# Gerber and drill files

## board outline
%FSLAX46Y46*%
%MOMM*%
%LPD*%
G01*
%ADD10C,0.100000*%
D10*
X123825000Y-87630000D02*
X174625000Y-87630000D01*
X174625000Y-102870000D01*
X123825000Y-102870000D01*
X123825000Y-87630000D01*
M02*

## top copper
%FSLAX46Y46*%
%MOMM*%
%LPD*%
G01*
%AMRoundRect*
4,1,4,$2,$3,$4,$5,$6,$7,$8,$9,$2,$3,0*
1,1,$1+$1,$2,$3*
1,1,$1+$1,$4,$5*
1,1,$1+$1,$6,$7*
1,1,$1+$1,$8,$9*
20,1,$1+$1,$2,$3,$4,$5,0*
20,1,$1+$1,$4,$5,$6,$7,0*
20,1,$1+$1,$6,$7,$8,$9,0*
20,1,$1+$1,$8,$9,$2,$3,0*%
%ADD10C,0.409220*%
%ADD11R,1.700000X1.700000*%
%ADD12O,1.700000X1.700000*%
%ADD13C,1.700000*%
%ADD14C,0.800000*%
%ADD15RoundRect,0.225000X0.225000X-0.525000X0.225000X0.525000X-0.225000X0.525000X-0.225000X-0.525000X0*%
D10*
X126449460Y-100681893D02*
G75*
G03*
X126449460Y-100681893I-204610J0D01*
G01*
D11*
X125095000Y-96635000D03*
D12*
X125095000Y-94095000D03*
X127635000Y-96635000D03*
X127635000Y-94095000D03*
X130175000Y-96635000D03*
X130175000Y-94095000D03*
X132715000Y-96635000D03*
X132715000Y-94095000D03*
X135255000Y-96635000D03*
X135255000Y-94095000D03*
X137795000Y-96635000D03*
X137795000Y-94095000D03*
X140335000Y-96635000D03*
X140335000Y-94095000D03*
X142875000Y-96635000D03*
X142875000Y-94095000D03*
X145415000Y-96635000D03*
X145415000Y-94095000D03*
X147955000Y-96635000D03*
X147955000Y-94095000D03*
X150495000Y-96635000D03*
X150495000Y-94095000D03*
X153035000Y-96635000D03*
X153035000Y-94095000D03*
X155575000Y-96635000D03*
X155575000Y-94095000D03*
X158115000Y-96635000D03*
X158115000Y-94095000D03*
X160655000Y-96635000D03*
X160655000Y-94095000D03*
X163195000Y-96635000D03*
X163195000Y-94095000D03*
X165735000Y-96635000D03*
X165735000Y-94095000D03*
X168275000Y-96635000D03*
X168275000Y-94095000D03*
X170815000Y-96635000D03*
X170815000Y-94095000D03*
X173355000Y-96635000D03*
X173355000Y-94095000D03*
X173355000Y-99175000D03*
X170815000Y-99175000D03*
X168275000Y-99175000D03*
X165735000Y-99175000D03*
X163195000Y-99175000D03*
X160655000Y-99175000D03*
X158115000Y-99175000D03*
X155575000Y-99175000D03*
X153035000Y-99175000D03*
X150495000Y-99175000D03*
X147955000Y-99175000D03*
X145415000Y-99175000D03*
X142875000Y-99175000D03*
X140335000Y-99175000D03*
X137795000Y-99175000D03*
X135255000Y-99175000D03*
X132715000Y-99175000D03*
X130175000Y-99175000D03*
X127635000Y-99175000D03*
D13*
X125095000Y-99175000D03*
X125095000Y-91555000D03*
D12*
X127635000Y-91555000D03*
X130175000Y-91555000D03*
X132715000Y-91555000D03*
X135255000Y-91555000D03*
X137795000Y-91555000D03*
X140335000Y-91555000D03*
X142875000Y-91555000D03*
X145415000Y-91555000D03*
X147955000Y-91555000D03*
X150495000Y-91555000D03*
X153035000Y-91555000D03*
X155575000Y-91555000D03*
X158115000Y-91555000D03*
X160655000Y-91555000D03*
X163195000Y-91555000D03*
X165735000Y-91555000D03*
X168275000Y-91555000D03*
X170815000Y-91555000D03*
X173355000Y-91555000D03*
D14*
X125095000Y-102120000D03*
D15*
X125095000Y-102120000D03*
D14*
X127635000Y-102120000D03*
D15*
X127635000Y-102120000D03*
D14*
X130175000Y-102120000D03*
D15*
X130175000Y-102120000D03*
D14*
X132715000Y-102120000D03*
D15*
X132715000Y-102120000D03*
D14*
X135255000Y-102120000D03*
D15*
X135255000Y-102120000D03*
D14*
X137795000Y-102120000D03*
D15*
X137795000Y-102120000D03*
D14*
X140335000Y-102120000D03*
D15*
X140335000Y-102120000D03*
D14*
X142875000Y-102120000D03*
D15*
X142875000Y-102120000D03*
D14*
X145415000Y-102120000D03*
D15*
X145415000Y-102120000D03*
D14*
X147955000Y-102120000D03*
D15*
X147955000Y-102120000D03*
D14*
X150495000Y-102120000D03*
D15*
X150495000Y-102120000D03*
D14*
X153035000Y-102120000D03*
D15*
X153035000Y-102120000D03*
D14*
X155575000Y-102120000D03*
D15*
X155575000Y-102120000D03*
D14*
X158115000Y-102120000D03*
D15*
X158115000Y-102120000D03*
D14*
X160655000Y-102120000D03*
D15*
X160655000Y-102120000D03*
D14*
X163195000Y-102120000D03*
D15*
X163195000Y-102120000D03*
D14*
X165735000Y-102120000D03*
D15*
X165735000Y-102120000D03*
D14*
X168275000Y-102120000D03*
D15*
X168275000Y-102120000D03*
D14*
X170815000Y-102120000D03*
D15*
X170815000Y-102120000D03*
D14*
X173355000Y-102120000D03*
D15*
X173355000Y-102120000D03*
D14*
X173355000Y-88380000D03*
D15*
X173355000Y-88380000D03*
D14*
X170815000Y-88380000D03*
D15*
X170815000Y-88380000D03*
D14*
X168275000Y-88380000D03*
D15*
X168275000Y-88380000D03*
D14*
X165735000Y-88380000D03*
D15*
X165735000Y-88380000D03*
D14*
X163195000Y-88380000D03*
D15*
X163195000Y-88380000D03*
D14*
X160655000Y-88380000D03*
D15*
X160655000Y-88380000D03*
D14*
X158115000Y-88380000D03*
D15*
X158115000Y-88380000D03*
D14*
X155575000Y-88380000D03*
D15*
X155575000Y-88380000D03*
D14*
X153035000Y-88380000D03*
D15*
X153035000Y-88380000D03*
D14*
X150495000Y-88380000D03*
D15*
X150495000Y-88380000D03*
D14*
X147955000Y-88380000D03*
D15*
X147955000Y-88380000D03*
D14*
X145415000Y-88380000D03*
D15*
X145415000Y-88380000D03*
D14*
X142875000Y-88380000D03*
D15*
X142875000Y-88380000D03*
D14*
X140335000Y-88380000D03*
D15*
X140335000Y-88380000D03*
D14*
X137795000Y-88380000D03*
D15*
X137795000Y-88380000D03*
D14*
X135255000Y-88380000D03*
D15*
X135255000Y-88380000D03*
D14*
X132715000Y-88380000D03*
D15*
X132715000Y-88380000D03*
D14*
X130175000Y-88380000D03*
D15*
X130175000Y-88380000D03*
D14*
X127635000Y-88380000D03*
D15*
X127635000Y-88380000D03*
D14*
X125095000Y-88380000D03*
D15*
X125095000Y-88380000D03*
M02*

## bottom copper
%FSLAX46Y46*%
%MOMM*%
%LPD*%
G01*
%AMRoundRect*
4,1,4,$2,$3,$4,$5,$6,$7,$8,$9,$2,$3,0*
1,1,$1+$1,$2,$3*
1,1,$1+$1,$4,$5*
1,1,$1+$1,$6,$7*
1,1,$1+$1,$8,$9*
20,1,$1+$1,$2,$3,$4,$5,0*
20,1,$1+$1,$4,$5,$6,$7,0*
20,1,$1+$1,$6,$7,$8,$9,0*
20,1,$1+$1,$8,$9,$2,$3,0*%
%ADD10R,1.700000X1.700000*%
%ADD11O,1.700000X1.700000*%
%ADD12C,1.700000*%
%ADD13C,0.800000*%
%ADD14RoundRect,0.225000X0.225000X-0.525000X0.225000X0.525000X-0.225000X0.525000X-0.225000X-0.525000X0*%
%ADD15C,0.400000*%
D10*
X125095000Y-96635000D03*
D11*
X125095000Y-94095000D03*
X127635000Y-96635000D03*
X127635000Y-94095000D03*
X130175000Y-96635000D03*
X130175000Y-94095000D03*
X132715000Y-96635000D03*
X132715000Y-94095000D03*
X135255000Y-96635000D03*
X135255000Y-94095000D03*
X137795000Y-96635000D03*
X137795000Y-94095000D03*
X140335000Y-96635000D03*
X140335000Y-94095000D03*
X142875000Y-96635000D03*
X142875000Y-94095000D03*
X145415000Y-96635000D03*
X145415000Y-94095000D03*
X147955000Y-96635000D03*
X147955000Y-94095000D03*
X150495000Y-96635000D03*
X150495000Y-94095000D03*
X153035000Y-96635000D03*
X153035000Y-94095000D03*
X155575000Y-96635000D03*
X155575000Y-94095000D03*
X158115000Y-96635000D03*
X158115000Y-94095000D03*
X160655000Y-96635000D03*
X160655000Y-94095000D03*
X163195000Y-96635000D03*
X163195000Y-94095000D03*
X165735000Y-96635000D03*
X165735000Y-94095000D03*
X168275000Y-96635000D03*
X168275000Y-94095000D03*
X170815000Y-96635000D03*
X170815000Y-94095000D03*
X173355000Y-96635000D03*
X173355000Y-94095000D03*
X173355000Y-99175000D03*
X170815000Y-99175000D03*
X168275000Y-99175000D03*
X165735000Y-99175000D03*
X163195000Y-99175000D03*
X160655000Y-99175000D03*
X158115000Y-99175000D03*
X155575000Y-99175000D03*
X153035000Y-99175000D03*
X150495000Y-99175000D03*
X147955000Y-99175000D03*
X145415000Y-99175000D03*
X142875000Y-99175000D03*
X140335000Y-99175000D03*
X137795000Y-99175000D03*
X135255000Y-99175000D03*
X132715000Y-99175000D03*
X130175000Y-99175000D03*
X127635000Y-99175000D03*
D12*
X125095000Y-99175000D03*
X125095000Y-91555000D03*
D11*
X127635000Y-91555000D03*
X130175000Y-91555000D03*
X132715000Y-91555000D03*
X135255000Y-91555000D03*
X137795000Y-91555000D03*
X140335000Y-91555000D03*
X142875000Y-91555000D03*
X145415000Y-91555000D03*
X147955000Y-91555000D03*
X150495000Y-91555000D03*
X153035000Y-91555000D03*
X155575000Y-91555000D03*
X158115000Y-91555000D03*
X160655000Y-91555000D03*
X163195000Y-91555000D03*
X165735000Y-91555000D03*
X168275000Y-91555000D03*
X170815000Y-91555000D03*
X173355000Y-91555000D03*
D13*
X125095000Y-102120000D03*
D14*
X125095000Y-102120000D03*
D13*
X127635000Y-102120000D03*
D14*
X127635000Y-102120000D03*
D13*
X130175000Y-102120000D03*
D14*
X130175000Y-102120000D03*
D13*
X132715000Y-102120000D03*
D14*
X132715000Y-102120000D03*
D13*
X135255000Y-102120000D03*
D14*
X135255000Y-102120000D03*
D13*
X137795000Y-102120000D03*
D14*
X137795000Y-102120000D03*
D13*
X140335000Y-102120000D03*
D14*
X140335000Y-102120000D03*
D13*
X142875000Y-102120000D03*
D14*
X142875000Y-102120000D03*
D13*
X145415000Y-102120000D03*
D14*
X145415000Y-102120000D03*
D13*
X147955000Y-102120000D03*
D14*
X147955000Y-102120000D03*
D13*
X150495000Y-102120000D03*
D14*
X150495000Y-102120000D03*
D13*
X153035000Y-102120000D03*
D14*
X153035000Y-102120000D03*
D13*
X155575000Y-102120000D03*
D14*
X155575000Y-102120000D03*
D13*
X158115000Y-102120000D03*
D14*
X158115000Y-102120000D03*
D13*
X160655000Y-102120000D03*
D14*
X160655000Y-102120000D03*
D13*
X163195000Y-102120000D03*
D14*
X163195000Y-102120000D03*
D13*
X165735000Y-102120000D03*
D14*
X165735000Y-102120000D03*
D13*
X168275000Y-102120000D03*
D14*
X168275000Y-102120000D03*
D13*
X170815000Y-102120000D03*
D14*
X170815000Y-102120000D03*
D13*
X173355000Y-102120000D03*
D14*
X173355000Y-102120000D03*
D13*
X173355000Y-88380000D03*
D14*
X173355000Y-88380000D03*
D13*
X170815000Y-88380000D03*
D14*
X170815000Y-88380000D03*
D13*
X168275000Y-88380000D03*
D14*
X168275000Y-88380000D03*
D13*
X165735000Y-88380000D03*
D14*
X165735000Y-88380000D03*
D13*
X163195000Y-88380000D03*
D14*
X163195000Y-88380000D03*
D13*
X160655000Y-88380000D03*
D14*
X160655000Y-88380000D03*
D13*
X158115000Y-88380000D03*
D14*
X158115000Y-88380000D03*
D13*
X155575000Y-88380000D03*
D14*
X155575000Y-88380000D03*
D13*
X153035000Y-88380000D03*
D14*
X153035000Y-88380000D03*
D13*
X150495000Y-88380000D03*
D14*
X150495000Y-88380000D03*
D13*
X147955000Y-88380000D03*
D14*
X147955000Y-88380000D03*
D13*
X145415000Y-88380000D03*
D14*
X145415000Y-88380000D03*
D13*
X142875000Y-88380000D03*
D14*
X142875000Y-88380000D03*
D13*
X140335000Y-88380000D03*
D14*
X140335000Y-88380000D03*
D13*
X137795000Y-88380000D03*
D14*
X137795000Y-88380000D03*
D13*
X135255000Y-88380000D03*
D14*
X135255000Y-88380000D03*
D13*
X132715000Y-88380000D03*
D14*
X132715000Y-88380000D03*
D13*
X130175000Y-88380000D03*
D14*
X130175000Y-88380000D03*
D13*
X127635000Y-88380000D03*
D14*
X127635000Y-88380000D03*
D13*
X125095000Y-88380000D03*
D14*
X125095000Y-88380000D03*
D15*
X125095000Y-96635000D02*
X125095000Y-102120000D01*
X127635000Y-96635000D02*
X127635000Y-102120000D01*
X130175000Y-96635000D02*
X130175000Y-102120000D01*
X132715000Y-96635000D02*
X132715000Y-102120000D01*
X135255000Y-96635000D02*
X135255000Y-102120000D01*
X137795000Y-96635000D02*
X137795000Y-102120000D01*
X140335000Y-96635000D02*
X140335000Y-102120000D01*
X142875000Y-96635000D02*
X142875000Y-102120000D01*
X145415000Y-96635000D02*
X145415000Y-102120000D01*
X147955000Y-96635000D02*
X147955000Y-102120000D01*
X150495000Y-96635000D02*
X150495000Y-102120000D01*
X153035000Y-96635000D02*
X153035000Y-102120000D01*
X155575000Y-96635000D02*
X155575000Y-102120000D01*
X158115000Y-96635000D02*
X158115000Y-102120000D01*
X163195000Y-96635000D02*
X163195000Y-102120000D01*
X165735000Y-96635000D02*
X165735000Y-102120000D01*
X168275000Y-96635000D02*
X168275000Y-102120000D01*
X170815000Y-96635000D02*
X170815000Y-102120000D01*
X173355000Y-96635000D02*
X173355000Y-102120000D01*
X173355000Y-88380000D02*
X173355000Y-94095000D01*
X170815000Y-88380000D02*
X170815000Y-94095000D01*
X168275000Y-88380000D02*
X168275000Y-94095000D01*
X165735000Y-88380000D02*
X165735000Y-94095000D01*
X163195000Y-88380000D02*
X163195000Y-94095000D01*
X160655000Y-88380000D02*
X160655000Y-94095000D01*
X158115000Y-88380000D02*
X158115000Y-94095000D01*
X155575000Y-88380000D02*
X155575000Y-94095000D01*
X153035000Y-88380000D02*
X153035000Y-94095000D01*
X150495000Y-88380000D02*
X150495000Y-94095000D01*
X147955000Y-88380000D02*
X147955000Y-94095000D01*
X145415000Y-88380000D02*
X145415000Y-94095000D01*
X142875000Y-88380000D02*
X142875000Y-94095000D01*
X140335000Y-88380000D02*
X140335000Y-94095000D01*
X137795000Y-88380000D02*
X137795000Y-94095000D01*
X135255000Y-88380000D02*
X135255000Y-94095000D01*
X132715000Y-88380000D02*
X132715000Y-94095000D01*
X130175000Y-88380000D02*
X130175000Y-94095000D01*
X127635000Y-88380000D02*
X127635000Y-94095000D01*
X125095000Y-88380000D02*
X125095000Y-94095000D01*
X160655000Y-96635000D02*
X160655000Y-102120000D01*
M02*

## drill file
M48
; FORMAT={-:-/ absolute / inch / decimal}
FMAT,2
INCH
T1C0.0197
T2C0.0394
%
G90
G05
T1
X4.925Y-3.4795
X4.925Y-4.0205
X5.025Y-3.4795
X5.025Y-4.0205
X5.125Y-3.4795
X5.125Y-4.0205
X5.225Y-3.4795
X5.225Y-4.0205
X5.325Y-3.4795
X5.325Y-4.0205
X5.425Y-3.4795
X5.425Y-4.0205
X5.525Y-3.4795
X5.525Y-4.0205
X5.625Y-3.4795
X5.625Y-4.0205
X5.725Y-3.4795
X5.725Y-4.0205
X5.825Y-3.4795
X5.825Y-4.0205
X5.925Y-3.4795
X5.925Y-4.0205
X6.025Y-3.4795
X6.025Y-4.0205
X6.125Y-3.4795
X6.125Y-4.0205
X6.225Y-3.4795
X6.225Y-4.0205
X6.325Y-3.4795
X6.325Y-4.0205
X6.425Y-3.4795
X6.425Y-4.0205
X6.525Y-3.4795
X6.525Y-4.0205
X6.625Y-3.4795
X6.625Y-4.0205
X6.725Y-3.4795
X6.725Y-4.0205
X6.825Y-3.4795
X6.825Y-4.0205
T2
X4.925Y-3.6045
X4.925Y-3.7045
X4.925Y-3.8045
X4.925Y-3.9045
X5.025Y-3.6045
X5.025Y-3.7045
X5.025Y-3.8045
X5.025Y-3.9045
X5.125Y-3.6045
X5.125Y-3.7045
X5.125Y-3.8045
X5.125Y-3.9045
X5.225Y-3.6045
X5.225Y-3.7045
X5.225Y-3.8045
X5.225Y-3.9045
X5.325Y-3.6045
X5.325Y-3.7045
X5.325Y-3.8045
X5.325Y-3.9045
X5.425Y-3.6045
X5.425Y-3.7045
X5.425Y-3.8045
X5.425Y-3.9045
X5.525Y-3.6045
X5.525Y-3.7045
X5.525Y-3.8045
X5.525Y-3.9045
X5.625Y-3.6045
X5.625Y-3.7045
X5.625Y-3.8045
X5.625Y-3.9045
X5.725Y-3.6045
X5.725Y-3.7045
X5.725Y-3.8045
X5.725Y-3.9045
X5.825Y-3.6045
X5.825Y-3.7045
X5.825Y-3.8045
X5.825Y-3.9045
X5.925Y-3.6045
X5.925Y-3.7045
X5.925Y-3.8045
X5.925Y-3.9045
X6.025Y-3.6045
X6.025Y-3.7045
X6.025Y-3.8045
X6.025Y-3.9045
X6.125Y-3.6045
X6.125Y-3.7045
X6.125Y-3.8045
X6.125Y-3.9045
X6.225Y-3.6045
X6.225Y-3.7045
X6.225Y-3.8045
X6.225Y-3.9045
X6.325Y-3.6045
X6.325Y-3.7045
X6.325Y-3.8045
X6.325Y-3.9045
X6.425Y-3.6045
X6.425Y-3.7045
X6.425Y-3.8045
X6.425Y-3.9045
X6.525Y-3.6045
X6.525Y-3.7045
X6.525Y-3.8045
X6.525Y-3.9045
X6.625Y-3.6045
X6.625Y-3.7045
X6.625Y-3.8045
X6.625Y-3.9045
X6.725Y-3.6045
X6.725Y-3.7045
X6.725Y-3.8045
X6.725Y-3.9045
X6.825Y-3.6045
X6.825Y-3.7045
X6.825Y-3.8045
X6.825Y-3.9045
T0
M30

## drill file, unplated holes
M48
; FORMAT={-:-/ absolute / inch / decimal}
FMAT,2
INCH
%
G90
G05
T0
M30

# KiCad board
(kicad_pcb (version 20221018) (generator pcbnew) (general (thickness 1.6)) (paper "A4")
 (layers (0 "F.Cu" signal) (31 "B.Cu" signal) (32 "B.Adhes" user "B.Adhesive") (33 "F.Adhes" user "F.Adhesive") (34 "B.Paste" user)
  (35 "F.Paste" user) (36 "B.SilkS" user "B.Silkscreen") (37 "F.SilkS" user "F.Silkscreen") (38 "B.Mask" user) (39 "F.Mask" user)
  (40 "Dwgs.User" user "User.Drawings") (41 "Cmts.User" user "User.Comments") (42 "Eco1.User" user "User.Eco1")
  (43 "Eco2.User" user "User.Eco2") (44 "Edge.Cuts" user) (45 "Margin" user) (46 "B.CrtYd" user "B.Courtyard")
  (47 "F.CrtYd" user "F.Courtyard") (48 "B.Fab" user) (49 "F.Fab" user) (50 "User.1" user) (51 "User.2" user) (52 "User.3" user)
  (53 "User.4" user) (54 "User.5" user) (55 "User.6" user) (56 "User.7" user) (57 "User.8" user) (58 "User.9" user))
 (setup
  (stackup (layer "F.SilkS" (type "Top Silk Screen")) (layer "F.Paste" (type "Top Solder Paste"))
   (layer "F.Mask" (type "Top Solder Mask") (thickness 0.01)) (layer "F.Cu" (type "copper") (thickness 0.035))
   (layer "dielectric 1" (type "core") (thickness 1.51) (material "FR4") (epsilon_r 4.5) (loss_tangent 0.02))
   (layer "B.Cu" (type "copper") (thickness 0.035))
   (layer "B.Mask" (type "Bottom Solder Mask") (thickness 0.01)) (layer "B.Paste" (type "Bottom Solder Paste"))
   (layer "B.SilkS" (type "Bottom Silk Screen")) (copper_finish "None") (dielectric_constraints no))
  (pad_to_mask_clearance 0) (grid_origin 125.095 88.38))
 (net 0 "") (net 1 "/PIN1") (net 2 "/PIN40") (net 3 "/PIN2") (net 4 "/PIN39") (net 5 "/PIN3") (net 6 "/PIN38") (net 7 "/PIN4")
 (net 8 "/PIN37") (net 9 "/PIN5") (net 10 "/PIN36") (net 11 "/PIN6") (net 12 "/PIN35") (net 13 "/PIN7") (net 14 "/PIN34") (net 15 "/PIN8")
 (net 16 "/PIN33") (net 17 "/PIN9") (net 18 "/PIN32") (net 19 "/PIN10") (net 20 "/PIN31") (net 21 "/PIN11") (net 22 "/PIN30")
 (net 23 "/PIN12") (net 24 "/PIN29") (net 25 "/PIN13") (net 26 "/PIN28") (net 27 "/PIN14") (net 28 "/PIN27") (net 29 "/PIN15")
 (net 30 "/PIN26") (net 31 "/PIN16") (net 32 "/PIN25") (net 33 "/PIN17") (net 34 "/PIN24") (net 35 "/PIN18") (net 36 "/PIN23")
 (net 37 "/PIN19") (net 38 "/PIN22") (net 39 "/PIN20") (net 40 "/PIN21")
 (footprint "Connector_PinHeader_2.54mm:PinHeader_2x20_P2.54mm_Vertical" (layer "F.Cu") (at 125.095 96.635 90)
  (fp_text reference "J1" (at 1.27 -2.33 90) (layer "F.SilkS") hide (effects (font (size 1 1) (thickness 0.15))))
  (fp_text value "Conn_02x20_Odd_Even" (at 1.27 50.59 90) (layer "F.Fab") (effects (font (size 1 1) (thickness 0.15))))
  (pad "1" thru_hole rect (at 0 0 90) (size 1.7 1.7) (drill 1) (layers "*.Cu" "*.Mask") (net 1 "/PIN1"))
  (pad "2" thru_hole oval (at 2.54 0 90) (size 1.7 1.7) (drill 1) (layers "*.Cu" "*.Mask") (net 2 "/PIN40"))
  (pad "3" thru_hole oval (at 0 2.54 90) (size 1.7 1.7) (drill 1) (layers "*.Cu" "*.Mask") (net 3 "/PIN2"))
  (pad "4" thru_hole oval (at 2.54 2.54 90) (size 1.7 1.7) (drill 1) (layers "*.Cu" "*.Mask") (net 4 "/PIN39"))
  (pad "5" thru_hole oval (at 0 5.08 90) (size 1.7 1.7) (drill 1) (layers "*.Cu" "*.Mask") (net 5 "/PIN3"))
  (pad "6" thru_hole oval (at 2.54 5.08 90) (size 1.7 1.7) (drill 1) (layers "*.Cu" "*.Mask") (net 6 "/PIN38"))
  (pad "7" thru_hole oval (at 0 7.62 90) (size 1.7 1.7) (drill 1) (layers "*.Cu" "*.Mask") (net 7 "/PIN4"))
  (pad "8" thru_hole oval (at 2.54 7.62 90) (size 1.7 1.7) (drill 1) (layers "*.Cu" "*.Mask") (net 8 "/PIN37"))
  (pad "9" thru_hole oval (at 0 10.16 90) (size 1.7 1.7) (drill 1) (layers "*.Cu" "*.Mask") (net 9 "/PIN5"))
  (pad "10" thru_hole oval (at 2.54 10.16 90) (size 1.7 1.7) (drill 1) (layers "*.Cu" "*.Mask") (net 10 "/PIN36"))
  (pad "11" thru_hole oval (at 0 12.7 90) (size 1.7 1.7) (drill 1) (layers "*.Cu" "*.Mask") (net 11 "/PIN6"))
  (pad "12" thru_hole oval (at 2.54 12.7 90) (size 1.7 1.7) (drill 1) (layers "*.Cu" "*.Mask") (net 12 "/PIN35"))
  (pad "13" thru_hole oval (at 0 15.24 90) (size 1.7 1.7) (drill 1) (layers "*.Cu" "*.Mask") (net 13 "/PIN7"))
  (pad "14" thru_hole oval (at 2.54 15.24 90) (size 1.7 1.7) (drill 1) (layers "*.Cu" "*.Mask") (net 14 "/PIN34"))
  (pad "15" thru_hole oval (at 0 17.78 90) (size 1.7 1.7) (drill 1) (layers "*.Cu" "*.Mask") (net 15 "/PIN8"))
  (pad "16" thru_hole oval (at 2.54 17.78 90) (size 1.7 1.7) (drill 1) (layers "*.Cu" "*.Mask") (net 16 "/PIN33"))
  (pad "17" thru_hole oval (at 0 20.32 90) (size 1.7 1.7) (drill 1) (layers "*.Cu" "*.Mask") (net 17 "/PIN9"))
  (pad "18" thru_hole oval (at 2.54 20.32 90) (size 1.7 1.7) (drill 1) (layers "*.Cu" "*.Mask") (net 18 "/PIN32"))
  (pad "19" thru_hole oval (at 0 22.86 90) (size 1.7 1.7) (drill 1) (layers "*.Cu" "*.Mask") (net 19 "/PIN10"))
  (pad "20" thru_hole oval (at 2.54 22.86 90) (size 1.7 1.7) (drill 1) (layers "*.Cu" "*.Mask") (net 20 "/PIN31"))
  (pad "21" thru_hole oval (at 0 25.4 90) (size 1.7 1.7) (drill 1) (layers "*.Cu" "*.Mask") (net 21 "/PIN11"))
  (pad "22" thru_hole oval (at 2.54 25.4 90) (size 1.7 1.7) (drill 1) (layers "*.Cu" "*.Mask") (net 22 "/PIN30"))
  (pad "23" thru_hole oval (at 0 27.94 90) (size 1.7 1.7) (drill 1) (layers "*.Cu" "*.Mask") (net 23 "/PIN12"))
  (pad "24" thru_hole oval (at 2.54 27.94 90) (size 1.7 1.7) (drill 1) (layers "*.Cu" "*.Mask") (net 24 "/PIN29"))
  (pad "25" thru_hole oval (at 0 30.48 90) (size 1.7 1.7) (drill 1) (layers "*.Cu" "*.Mask") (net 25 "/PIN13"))
  (pad "26" thru_hole oval (at 2.54 30.48 90) (size 1.7 1.7) (drill 1) (layers "*.Cu" "*.Mask") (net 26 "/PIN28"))
  (pad "27" thru_hole oval (at 0 33.02 90) (size 1.7 1.7) (drill 1) (layers "*.Cu" "*.Mask") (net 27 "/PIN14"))
  (pad "28" thru_hole oval (at 2.54 33.02 90) (size 1.7 1.7) (drill 1) (layers "*.Cu" "*.Mask") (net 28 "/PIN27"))
  (pad "29" thru_hole oval (at 0 35.56 90) (size 1.7 1.7) (drill 1) (layers "*.Cu" "*.Mask") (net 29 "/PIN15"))
  (pad "30" thru_hole oval (at 2.54 35.56 90) (size 1.7 1.7) (drill 1) (layers "*.Cu" "*.Mask") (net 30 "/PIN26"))
  (pad "31" thru_hole oval (at 0 38.1 90) (size 1.7 1.7) (drill 1) (layers "*.Cu" "*.Mask") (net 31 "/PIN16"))
  (pad "32" thru_hole oval (at 2.54 38.1 90) (size 1.7 1.7) (drill 1) (layers "*.Cu" "*.Mask") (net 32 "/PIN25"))
  (pad "33" thru_hole oval (at 0 40.64 90) (size 1.7 1.7) (drill 1) (layers "*.Cu" "*.Mask") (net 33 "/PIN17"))
  (pad "34" thru_hole oval (at 2.54 40.64 90) (size 1.7 1.7) (drill 1) (layers "*.Cu" "*.Mask") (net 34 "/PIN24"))
  (pad "35" thru_hole oval (at 0 43.18 90) (size 1.7 1.7) (drill 1) (layers "*.Cu" "*.Mask") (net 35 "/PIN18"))
  (pad "36" thru_hole oval (at 2.54 43.18 90) (size 1.7 1.7) (drill 1) (layers "*.Cu" "*.Mask") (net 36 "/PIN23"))
  (pad "37" thru_hole oval (at 0 45.72 90) (size 1.7 1.7) (drill 1) (layers "*.Cu" "*.Mask") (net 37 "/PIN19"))
  (pad "38" thru_hole oval (at 2.54 45.72 90) (size 1.7 1.7) (drill 1) (layers "*.Cu" "*.Mask") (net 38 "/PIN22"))
  (pad "39" thru_hole oval (at 0 48.26 90) (size 1.7 1.7) (drill 1) (layers "*.Cu" "*.Mask") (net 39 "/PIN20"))
  (pad "40" thru_hole oval (at 2.54 48.26 90) (size 1.7 1.7) (drill 1) (layers "*.Cu" "*.Mask") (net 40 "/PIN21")))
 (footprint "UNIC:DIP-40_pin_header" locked (layer "F.Cu") (at 149.225 95.25 90)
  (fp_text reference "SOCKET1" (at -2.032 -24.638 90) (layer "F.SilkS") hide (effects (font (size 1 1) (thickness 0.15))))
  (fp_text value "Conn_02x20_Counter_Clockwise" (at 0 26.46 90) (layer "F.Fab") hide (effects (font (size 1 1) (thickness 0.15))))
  (pad "1" thru_hole circle locked (at -6.87 -24.13 90) (size 0.8 0.8) (drill 0.5) (layers "*.Cu" "*.Mask") (remove_unused_layers)
   (keep_end_layers) (zone_layer_connections) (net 1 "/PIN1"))
  (pad "1" smd roundrect locked (at -6.87 -24.13 90) (size 1.5 0.9) (layers "F.Cu" "F.Paste" "F.Mask") (roundrect_rratio 0.25)
   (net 1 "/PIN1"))
  (pad "1" smd roundrect locked (at -6.87 -24.13 90) (size 1.5 0.9) (layers "B.Cu" "B.Paste" "B.Mask") (roundrect_rratio 0.25)
   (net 1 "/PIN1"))
  (pad "2" thru_hole circle locked (at -6.87 -21.59 90) (size 0.8 0.8) (drill 0.5) (layers "*.Cu" "*.Mask") (remove_unused_layers)
   (keep_end_layers) (zone_layer_connections) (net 3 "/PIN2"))
  (pad "2" smd roundrect locked (at -6.87 -21.59 90) (size 1.5 0.9) (layers "F.Cu" "F.Paste" "F.Mask") (roundrect_rratio 0.25)
   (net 3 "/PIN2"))
  (pad "2" smd roundrect locked (at -6.87 -21.59 90) (size 1.5 0.9) (layers "B.Cu" "B.Paste" "B.Mask") (roundrect_rratio 0.25)
   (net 3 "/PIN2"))
  (pad "3" thru_hole circle locked (at -6.87 -19.05 90) (size 0.8 0.8) (drill 0.5) (layers "*.Cu" "*.Mask") (remove_unused_layers)
   (keep_end_layers) (zone_layer_connections) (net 5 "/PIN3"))
  (pad "3" smd roundrect locked (at -6.87 -19.05 90) (size 1.5 0.9) (layers "F.Cu" "F.Paste" "F.Mask") (roundrect_rratio 0.25)
   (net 5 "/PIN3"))
  (pad "3" smd roundrect locked (at -6.87 -19.05 90) (size 1.5 0.9) (layers "B.Cu" "B.Paste" "B.Mask") (roundrect_rratio 0.25)
   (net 5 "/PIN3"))
  (pad "4" thru_hole circle locked (at -6.87 -16.51 90) (size 0.8 0.8) (drill 0.5) (layers "*.Cu" "*.Mask") (remove_unused_layers)
   (keep_end_layers) (zone_layer_connections) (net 7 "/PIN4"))
  (pad "4" smd roundrect locked (at -6.87 -16.51 90) (size 1.5 0.9) (layers "F.Cu" "F.Paste" "F.Mask") (roundrect_rratio 0.25)
   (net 7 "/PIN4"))
  (pad "4" smd roundrect locked (at -6.87 -16.51 90) (size 1.5 0.9) (layers "B.Cu" "B.Paste" "B.Mask") (roundrect_rratio 0.25)
   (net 7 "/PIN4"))
  (pad "5" thru_hole circle locked (at -6.87 -13.97 90) (size 0.8 0.8) (drill 0.5) (layers "*.Cu" "*.Mask") (remove_unused_layers)
   (keep_end_layers) (zone_layer_connections) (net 9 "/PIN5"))
  (pad "5" smd roundrect locked (at -6.87 -13.97 90) (size 1.5 0.9) (layers "F.Cu" "F.Paste" "F.Mask") (roundrect_rratio 0.25)
   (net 9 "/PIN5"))
  (pad "5" smd roundrect locked (at -6.87 -13.97 90) (size 1.5 0.9) (layers "B.Cu" "B.Paste" "B.Mask") (roundrect_rratio 0.25)
   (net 9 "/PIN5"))
  (pad "6" thru_hole circle locked (at -6.87 -11.43 90) (size 0.8 0.8) (drill 0.5) (layers "*.Cu" "*.Mask") (remove_unused_layers)
   (keep_end_layers) (zone_layer_connections) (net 11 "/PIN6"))
  (pad "6" smd roundrect locked (at -6.87 -11.43 90) (size 1.5 0.9) (layers "F.Cu" "F.Paste" "F.Mask") (roundrect_rratio 0.25)
   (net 11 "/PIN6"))
  (pad "6" smd roundrect locked (at -6.87 -11.43 90) (size 1.5 0.9) (layers "B.Cu" "B.Paste" "B.Mask") (roundrect_rratio 0.25)
   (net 11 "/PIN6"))
  (pad "7" thru_hole circle locked (at -6.87 -8.89 90) (size 0.8 0.8) (drill 0.5) (layers "*.Cu" "*.Mask") (remove_unused_layers)
   (keep_end_layers) (zone_layer_connections) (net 13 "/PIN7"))
  (pad "7" smd roundrect locked (at -6.87 -8.89 90) (size 1.5 0.9) (layers "F.Cu" "F.Paste" "F.Mask") (roundrect_rratio 0.25)
   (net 13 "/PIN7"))
  (pad "7" smd roundrect locked (at -6.87 -8.89 90) (size 1.5 0.9) (layers "B.Cu" "B.Paste" "B.Mask") (roundrect_rratio 0.25)
   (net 13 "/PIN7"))
  (pad "8" thru_hole circle locked (at -6.87 -6.35 90) (size 0.8 0.8) (drill 0.5) (layers "*.Cu" "*.Mask") (remove_unused_layers)
   (keep_end_layers) (zone_layer_connections) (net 15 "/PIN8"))
  (pad "8" smd roundrect locked (at -6.87 -6.35 90) (size 1.5 0.9) (layers "F.Cu" "F.Paste" "F.Mask") (roundrect_rratio 0.25)
   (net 15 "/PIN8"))
  (pad "8" smd roundrect locked (at -6.87 -6.35 90) (size 1.5 0.9) (layers "B.Cu" "B.Paste" "B.Mask") (roundrect_rratio 0.25)
   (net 15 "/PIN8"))
  (pad "9" thru_hole circle locked (at -6.87 -3.81 90) (size 0.8 0.8) (drill 0.5) (layers "*.Cu" "*.Mask") (remove_unused_layers)
   (keep_end_layers) (zone_layer_connections) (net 17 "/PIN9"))
  (pad "9" smd roundrect locked (at -6.87 -3.81 90) (size 1.5 0.9) (layers "F.Cu" "F.Paste" "F.Mask") (roundrect_rratio 0.25)
   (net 17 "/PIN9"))
  (pad "9" smd roundrect locked (at -6.87 -3.81 90) (size 1.5 0.9) (layers "B.Cu" "B.Paste" "B.Mask") (roundrect_rratio 0.25)
   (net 17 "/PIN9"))
  (pad "10" thru_hole circle locked (at -6.87 -1.27 90) (size 0.8 0.8) (drill 0.5) (layers "*.Cu" "*.Mask") (remove_unused_layers)
   (keep_end_layers) (zone_layer_connections) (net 19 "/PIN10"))
  (pad "10" smd roundrect locked (at -6.87 -1.27 90) (size 1.5 0.9) (layers "F.Cu" "F.Paste" "F.Mask") (roundrect_rratio 0.25)
   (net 19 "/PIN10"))
  (pad "10" smd roundrect locked (at -6.87 -1.27 90) (size 1.5 0.9) (layers "B.Cu" "B.Paste" "B.Mask") (roundrect_rratio 0.25)
   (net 19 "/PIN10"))
  (pad "11" thru_hole circle locked (at -6.87 1.27 90) (size 0.8 0.8) (drill 0.5) (layers "*.Cu" "*.Mask") (remove_unused_layers)
   (keep_end_layers) (zone_layer_connections) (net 21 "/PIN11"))
  (pad "11" smd roundrect locked (at -6.87 1.27 90) (size 1.5 0.9) (layers "F.Cu" "F.Paste" "F.Mask") (roundrect_rratio 0.25)
   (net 21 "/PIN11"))
  (pad "11" smd roundrect locked (at -6.87 1.27 90) (size 1.5 0.9) (layers "B.Cu" "B.Paste" "B.Mask") (roundrect_rratio 0.25)
   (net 21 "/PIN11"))
  (pad "12" thru_hole circle locked (at -6.87 3.81 90) (size 0.8 0.8) (drill 0.5) (layers "*.Cu" "*.Mask") (remove_unused_layers)
   (keep_end_layers) (zone_layer_connections) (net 23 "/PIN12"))
  (pad "12" smd roundrect locked (at -6.87 3.81 90) (size 1.5 0.9) (layers "F.Cu" "F.Paste" "F.Mask") (roundrect_rratio 0.25)
   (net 23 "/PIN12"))
  (pad "12" smd roundrect locked (at -6.87 3.81 90) (size 1.5 0.9) (layers "B.Cu" "B.Paste" "B.Mask") (roundrect_rratio 0.25)
   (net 23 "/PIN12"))
  (pad "13" thru_hole circle locked (at -6.87 6.35 90) (size 0.8 0.8) (drill 0.5) (layers "*.Cu" "*.Mask") (remove_unused_layers)
   (keep_end_layers) (zone_layer_connections) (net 25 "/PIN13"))
  (pad "13" smd roundrect locked (at -6.87 6.35 90) (size 1.5 0.9) (layers "F.Cu" "F.Paste" "F.Mask") (roundrect_rratio 0.25)
   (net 25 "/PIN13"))
  (pad "13" smd roundrect locked (at -6.87 6.35 90) (size 1.5 0.9) (layers "B.Cu" "B.Paste" "B.Mask") (roundrect_rratio 0.25)
   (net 25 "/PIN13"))
  (pad "14" thru_hole circle locked (at -6.87 8.89 90) (size 0.8 0.8) (drill 0.5) (layers "*.Cu" "*.Mask") (remove_unused_layers)
   (keep_end_layers) (zone_layer_connections) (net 27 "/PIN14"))
  (pad "14" smd roundrect locked (at -6.87 8.89 90) (size 1.5 0.9) (layers "F.Cu" "F.Paste" "F.Mask") (roundrect_rratio 0.25)
   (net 27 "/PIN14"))
  (pad "14" smd roundrect locked (at -6.87 8.89 90) (size 1.5 0.9) (layers "B.Cu" "B.Paste" "B.Mask") (roundrect_rratio 0.25)
   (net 27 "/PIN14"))
  (pad "15" thru_hole circle locked (at -6.87 11.43 90) (size 0.8 0.8) (drill 0.5) (layers "*.Cu" "*.Mask") (remove_unused_layers)
   (keep_end_layers) (zone_layer_connections) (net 29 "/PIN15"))
  (pad "15" smd roundrect locked (at -6.87 11.43 90) (size 1.5 0.9) (layers "F.Cu" "F.Paste" "F.Mask") (roundrect_rratio 0.25)
   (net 29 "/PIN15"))
  (pad "15" smd roundrect locked (at -6.87 11.43 90) (size 1.5 0.9) (layers "B.Cu" "B.Paste" "B.Mask") (roundrect_rratio 0.25)
   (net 29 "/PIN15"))
  (pad "16" thru_hole circle locked (at -6.87 13.97 90) (size 0.8 0.8) (drill 0.5) (layers "*.Cu" "*.Mask") (remove_unused_layers)
   (keep_end_layers) (zone_layer_connections) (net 31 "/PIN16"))
  (pad "16" smd roundrect locked (at -6.87 13.97 90) (size 1.5 0.9) (layers "F.Cu" "F.Paste" "F.Mask") (roundrect_rratio 0.25)
   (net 31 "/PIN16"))
  (pad "16" smd roundrect locked (at -6.87 13.97 90) (size 1.5 0.9) (layers "B.Cu" "B.Paste" "B.Mask") (roundrect_rratio 0.25)
   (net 31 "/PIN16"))
  (pad "17" thru_hole circle locked (at -6.87 16.51 90) (size 0.8 0.8) (drill 0.5) (layers "*.Cu" "*.Mask") (remove_unused_layers)
   (keep_end_layers) (zone_layer_connections) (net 33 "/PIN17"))
  (pad "17" smd roundrect locked (at -6.87 16.51 90) (size 1.5 0.9) (layers "F.Cu" "F.Paste" "F.Mask") (roundrect_rratio 0.25)
   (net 33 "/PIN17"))
  (pad "17" smd roundrect locked (at -6.87 16.51 90) (size 1.5 0.9) (layers "B.Cu" "B.Paste" "B.Mask") (roundrect_rratio 0.25)
   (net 33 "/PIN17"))
  (pad "18" thru_hole circle locked (at -6.87 19.05 90) (size 0.8 0.8) (drill 0.5) (layers "*.Cu" "*.Mask") (remove_unused_layers)
   (keep_end_layers) (zone_layer_connections) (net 35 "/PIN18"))
  (pad "18" smd roundrect locked (at -6.87 19.05 90) (size 1.5 0.9) (layers "F.Cu" "F.Paste" "F.Mask") (roundrect_rratio 0.25)
   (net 35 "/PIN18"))
  (pad "18" smd roundrect locked (at -6.87 19.05 90) (size 1.5 0.9) (layers "B.Cu" "B.Paste" "B.Mask") (roundrect_rratio 0.25)
   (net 35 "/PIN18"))
  (pad "19" thru_hole circle locked (at -6.87 21.59 90) (size 0.8 0.8) (drill 0.5) (layers "*.Cu" "*.Mask") (remove_unused_layers)
   (keep_end_layers) (zone_layer_connections) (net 37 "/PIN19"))
  (pad "19" smd roundrect locked (at -6.87 21.59 90) (size 1.5 0.9) (layers "F.Cu" "F.Paste" "F.Mask") (roundrect_rratio 0.25)
   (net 37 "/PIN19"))
  (pad "19" smd roundrect locked (at -6.87 21.59 90) (size 1.5 0.9) (layers "B.Cu" "B.Paste" "B.Mask") (roundrect_rratio 0.25)
   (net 37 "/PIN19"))
  (pad "20" thru_hole circle locked (at -6.87 24.13 90) (size 0.8 0.8) (drill 0.5) (layers "*.Cu" "*.Mask") (remove_unused_layers)
   (keep_end_layers) (zone_layer_connections) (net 39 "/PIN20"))
  (pad "20" smd roundrect locked (at -6.87 24.13 90) (size 1.5 0.9) (layers "F.Cu" "F.Paste" "F.Mask") (roundrect_rratio 0.25)
   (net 39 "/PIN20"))
  (pad "20" smd roundrect locked (at -6.87 24.13 90) (size 1.5 0.9) (layers "B.Cu" "B.Paste" "B.Mask") (roundrect_rratio 0.25)
   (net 39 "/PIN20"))
  (pad "21" thru_hole circle locked (at 6.87 24.13 90) (size 0.8 0.8) (drill 0.5) (layers "*.Cu" "*.Mask") (remove_unused_layers)
   (keep_end_layers) (zone_layer_connections) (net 40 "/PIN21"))
  (pad "21" smd roundrect locked (at 6.87 24.13 90) (size 1.5 0.9) (layers "F.Cu" "F.Paste" "F.Mask") (roundrect_rratio 0.25)
   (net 40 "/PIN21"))
  (pad "21" smd roundrect locked (at 6.87 24.13 90) (size 1.5 0.9) (layers "B.Cu" "B.Paste" "B.Mask") (roundrect_rratio 0.25)
   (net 40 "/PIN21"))
  (pad "22" thru_hole circle locked (at 6.87 21.59 90) (size 0.8 0.8) (drill 0.5) (layers "*.Cu" "*.Mask") (remove_unused_layers)
   (keep_end_layers) (zone_layer_connections) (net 38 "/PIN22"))
  (pad "22" smd roundrect locked (at 6.87 21.59 90) (size 1.5 0.9) (layers "F.Cu" "F.Paste" "F.Mask") (roundrect_rratio 0.25)
   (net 38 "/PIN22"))
  (pad "22" smd roundrect locked (at 6.87 21.59 90) (size 1.5 0.9) (layers "B.Cu" "B.Paste" "B.Mask") (roundrect_rratio 0.25)
   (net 38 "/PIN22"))
  (pad "23" thru_hole circle locked (at 6.87 19.05 90) (size 0.8 0.8) (drill 0.5) (layers "*.Cu" "*.Mask") (remove_unused_layers)
   (keep_end_layers) (zone_layer_connections) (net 36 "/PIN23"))
  (pad "23" smd roundrect locked (at 6.87 19.05 90) (size 1.5 0.9) (layers "F.Cu" "F.Paste" "F.Mask") (roundrect_rratio 0.25)
   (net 36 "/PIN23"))
  (pad "23" smd roundrect locked (at 6.87 19.05 90) (size 1.5 0.9) (layers "B.Cu" "B.Paste" "B.Mask") (roundrect_rratio 0.25)
   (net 36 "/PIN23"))
  (pad "24" thru_hole circle locked (at 6.87 16.51 90) (size 0.8 0.8) (drill 0.5) (layers "*.Cu" "*.Mask") (remove_unused_layers)
   (keep_end_layers) (zone_layer_connections) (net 34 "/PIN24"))
  (pad "24" smd roundrect locked (at 6.87 16.51 90) (size 1.5 0.9) (layers "F.Cu" "F.Paste" "F.Mask") (roundrect_rratio 0.25)
   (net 34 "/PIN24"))
  (pad "24" smd roundrect locked (at 6.87 16.51 90) (size 1.5 0.9) (layers "B.Cu" "B.Paste" "B.Mask") (roundrect_rratio 0.25)
   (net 34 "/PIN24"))
  (pad "25" thru_hole circle locked (at 6.87 13.97 90) (size 0.8 0.8) (drill 0.5) (layers "*.Cu" "*.Mask") (remove_unused_layers)
   (keep_end_layers) (zone_layer_connections) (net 32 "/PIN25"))
  (pad "25" smd roundrect locked (at 6.87 13.97 90) (size 1.5 0.9) (layers "F.Cu" "F.Paste" "F.Mask") (roundrect_rratio 0.25)
   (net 32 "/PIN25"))
  (pad "25" smd roundrect locked (at 6.87 13.97 90) (size 1.5 0.9) (layers "B.Cu" "B.Paste" "B.Mask") (roundrect_rratio 0.25)
   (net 32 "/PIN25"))
  (pad "26" thru_hole circle locked (at 6.87 11.43 90) (size 0.8 0.8) (drill 0.5) (layers "*.Cu" "*.Mask") (remove_unused_layers)
   (keep_end_layers) (zone_layer_connections) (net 30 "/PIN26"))
  (pad "26" smd roundrect locked (at 6.87 11.43 90) (size 1.5 0.9) (layers "F.Cu" "F.Paste" "F.Mask") (roundrect_rratio 0.25)
   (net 30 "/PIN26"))
  (pad "26" smd roundrect locked (at 6.87 11.43 90) (size 1.5 0.9) (layers "B.Cu" "B.Paste" "B.Mask") (roundrect_rratio 0.25)
   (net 30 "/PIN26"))
  (pad "27" thru_hole circle locked (at 6.87 8.89 90) (size 0.8 0.8) (drill 0.5) (layers "*.Cu" "*.Mask") (remove_unused_layers)
   (keep_end_layers) (zone_layer_connections) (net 28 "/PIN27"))
  (pad "27" smd roundrect locked (at 6.87 8.89 90) (size 1.5 0.9) (layers "F.Cu" "F.Paste" "F.Mask") (roundrect_rratio 0.25)
   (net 28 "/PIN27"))
  (pad "27" smd roundrect locked (at 6.87 8.89 90) (size 1.5 0.9) (layers "B.Cu" "B.Paste" "B.Mask") (roundrect_rratio 0.25)
   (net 28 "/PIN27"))
  (pad "28" thru_hole circle locked (at 6.87 6.35 90) (size 0.8 0.8) (drill 0.5) (layers "*.Cu" "*.Mask") (remove_unused_layers)
   (keep_end_layers) (zone_layer_connections) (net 26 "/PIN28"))
  (pad "28" smd roundrect locked (at 6.87 6.35 90) (size 1.5 0.9) (layers "F.Cu" "F.Paste" "F.Mask") (roundrect_rratio 0.25)
   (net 26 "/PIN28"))
  (pad "28" smd roundrect locked (at 6.87 6.35 90) (size 1.5 0.9) (layers "B.Cu" "B.Paste" "B.Mask") (roundrect_rratio 0.25)
   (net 26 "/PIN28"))
  (pad "29" thru_hole circle locked (at 6.87 3.81 90) (size 0.8 0.8) (drill 0.5) (layers "*.Cu" "*.Mask") (remove_unused_layers)
   (keep_end_layers) (zone_layer_connections) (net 24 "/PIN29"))
  (pad "29" smd roundrect locked (at 6.87 3.81 90) (size 1.5 0.9) (layers "F.Cu" "F.Paste" "F.Mask") (roundrect_rratio 0.25)
   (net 24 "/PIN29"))
  (pad "29" smd roundrect locked (at 6.87 3.81 90) (size 1.5 0.9) (layers "B.Cu" "B.Paste" "B.Mask") (roundrect_rratio 0.25)
   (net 24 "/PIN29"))
  (pad "30" thru_hole circle locked (at 6.87 1.27 90) (size 0.8 0.8) (drill 0.5) (layers "*.Cu" "*.Mask") (remove_unused_layers)
   (keep_end_layers) (zone_layer_connections) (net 22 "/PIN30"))
  (pad "30" smd roundrect locked (at 6.87 1.27 90) (size 1.5 0.9) (layers "F.Cu" "F.Paste" "F.Mask") (roundrect_rratio 0.25)
   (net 22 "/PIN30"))
  (pad "30" smd roundrect locked (at 6.87 1.27 90) (size 1.5 0.9) (layers "B.Cu" "B.Paste" "B.Mask") (roundrect_rratio 0.25)
   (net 22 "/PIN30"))
  (pad "31" thru_hole circle locked (at 6.87 -1.27 90) (size 0.8 0.8) (drill 0.5) (layers "*.Cu" "*.Mask") (remove_unused_layers)
   (keep_end_layers) (zone_layer_connections) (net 20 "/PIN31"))
  (pad "31" smd roundrect locked (at 6.87 -1.27 90) (size 1.5 0.9) (layers "F.Cu" "F.Paste" "F.Mask") (roundrect_rratio 0.25)
   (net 20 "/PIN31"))
  (pad "31" smd roundrect locked (at 6.87 -1.27 90) (size 1.5 0.9) (layers "B.Cu" "B.Paste" "B.Mask") (roundrect_rratio 0.25)
   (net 20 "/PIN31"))
  (pad "32" thru_hole circle locked (at 6.87 -3.81 90) (size 0.8 0.8) (drill 0.5) (layers "*.Cu" "*.Mask") (remove_unused_layers)
   (keep_end_layers) (zone_layer_connections) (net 18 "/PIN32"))
  (pad "32" smd roundrect locked (at 6.87 -3.81 90) (size 1.5 0.9) (layers "F.Cu" "F.Paste" "F.Mask") (roundrect_rratio 0.25)
   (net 18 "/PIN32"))
  (pad "32" smd roundrect locked (at 6.87 -3.81 90) (size 1.5 0.9) (layers "B.Cu" "B.Paste" "B.Mask") (roundrect_rratio 0.25)
   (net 18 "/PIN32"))
  (pad "33" thru_hole circle locked (at 6.87 -6.35 90) (size 0.8 0.8) (drill 0.5) (layers "*.Cu" "*.Mask") (remove_unused_layers)
   (keep_end_layers) (zone_layer_connections) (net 16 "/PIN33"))
  (pad "33" smd roundrect locked (at 6.87 -6.35 90) (size 1.5 0.9) (layers "F.Cu" "F.Paste" "F.Mask") (roundrect_rratio 0.25)
   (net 16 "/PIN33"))
  (pad "33" smd roundrect locked (at 6.87 -6.35 90) (size 1.5 0.9) (layers "B.Cu" "B.Paste" "B.Mask") (roundrect_rratio 0.25)
   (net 16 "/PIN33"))
  (pad "34" thru_hole circle locked (at 6.87 -8.89 90) (size 0.8 0.8) (drill 0.5) (layers "*.Cu" "*.Mask") (remove_unused_layers)
   (keep_end_layers) (zone_layer_connections) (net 14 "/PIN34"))
  (pad "34" smd roundrect locked (at 6.87 -8.89 90) (size 1.5 0.9) (layers "F.Cu" "F.Paste" "F.Mask") (roundrect_rratio 0.25)
   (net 14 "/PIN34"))
  (pad "34" smd roundrect locked (at 6.87 -8.89 90) (size 1.5 0.9) (layers "B.Cu" "B.Paste" "B.Mask") (roundrect_rratio 0.25)
   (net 14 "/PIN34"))
  (pad "35" thru_hole circle locked (at 6.87 -11.43 90) (size 0.8 0.8) (drill 0.5) (layers "*.Cu" "*.Mask") (remove_unused_layers)
   (keep_end_layers) (zone_layer_connections) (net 12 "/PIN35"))
  (pad "35" smd roundrect locked (at 6.87 -11.43 90) (size 1.5 0.9) (layers "F.Cu" "F.Paste" "F.Mask") (roundrect_rratio 0.25)
   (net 12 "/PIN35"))
  (pad "35" smd roundrect locked (at 6.87 -11.43 90) (size 1.5 0.9) (layers "B.Cu" "B.Paste" "B.Mask") (roundrect_rratio 0.25)
   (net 12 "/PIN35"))
  (pad "36" thru_hole circle locked (at 6.87 -13.97 90) (size 0.8 0.8) (drill 0.5) (layers "*.Cu" "*.Mask") (remove_unused_layers)
   (keep_end_layers) (zone_layer_connections) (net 10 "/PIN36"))
  (pad "36" smd roundrect locked (at 6.87 -13.97 90) (size 1.5 0.9) (layers "F.Cu" "F.Paste" "F.Mask") (roundrect_rratio 0.25)
   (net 10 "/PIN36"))
  (pad "36" smd roundrect locked (at 6.87 -13.97 90) (size 1.5 0.9) (layers "B.Cu" "B.Paste" "B.Mask") (roundrect_rratio 0.25)
   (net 10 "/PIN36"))
  (pad "37" thru_hole circle locked (at 6.87 -16.51 90) (size 0.8 0.8) (drill 0.5) (layers "*.Cu" "*.Mask") (remove_unused_layers)
   (keep_end_layers) (zone_layer_connections) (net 8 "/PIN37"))
  (pad "37" smd roundrect locked (at 6.87 -16.51 90) (size 1.5 0.9) (layers "F.Cu" "F.Paste" "F.Mask") (roundrect_rratio 0.25)
   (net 8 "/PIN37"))
  (pad "37" smd roundrect locked (at 6.87 -16.51 90) (size 1.5 0.9) (layers "B.Cu" "B.Paste" "B.Mask") (roundrect_rratio 0.25)
   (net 8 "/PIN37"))
  (pad "38" thru_hole circle locked (at 6.87 -19.05 90) (size 0.8 0.8) (drill 0.5) (layers "*.Cu" "*.Mask") (remove_unused_layers)
   (keep_end_layers) (zone_layer_connections) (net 6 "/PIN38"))
  (pad "38" smd roundrect locked (at 6.87 -19.05 90) (size 1.5 0.9) (layers "F.Cu" "F.Paste" "F.Mask") (roundrect_rratio 0.25)
   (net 6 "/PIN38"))
  (pad "38" smd roundrect locked (at 6.87 -19.05 90) (size 1.5 0.9) (layers "B.Cu" "B.Paste" "B.Mask") (roundrect_rratio 0.25)
   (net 6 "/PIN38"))
  (pad "39" thru_hole circle locked (at 6.87 -21.59 90) (size 0.8 0.8) (drill 0.5) (layers "*.Cu" "*.Mask") (remove_unused_layers)
   (keep_end_layers) (zone_layer_connections) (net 4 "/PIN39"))
  (pad "39" smd roundrect locked (at 6.87 -21.59 90) (size 1.5 0.9) (layers "F.Cu" "F.Paste" "F.Mask") (roundrect_rratio 0.25)
   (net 4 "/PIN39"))
  (pad "39" smd roundrect locked (at 6.87 -21.59 90) (size 1.5 0.9) (layers "B.Cu" "B.Paste" "B.Mask") (roundrect_rratio 0.25)
   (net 4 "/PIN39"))
  (pad "40" thru_hole circle locked (at 6.87 -24.13 90) (size 0.8 0.8) (drill 0.5) (layers "*.Cu" "*.Mask") (remove_unused_layers)
   (keep_end_layers) (zone_layer_connections) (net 2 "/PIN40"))
  (pad "40" smd roundrect locked (at 6.87 -24.13 90) (size 1.5 0.9) (layers "F.Cu" "F.Paste" "F.Mask") (roundrect_rratio 0.25)
   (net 2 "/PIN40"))
  (pad "40" smd roundrect locked (at 6.87 -24.13 90) (size 1.5 0.9) (layers "B.Cu" "B.Paste" "B.Mask") (roundrect_rratio 0.25)
   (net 2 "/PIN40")))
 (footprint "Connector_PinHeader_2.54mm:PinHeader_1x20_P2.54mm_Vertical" (layer "F.Cu") (at 125.095 91.555 90)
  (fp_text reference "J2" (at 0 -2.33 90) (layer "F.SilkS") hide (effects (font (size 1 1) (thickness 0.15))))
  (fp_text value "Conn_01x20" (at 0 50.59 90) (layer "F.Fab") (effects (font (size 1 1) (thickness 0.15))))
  (pad "1" thru_hole circle (at 0 0 90) (size 1.7 1.7) (drill 1) (layers "*.Cu" "*.Mask") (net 2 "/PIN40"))
  (pad "2" thru_hole oval (at 0 2.54 90) (size 1.7 1.7) (drill 1) (layers "*.Cu" "*.Mask") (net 4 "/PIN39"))
  (pad "3" thru_hole oval (at 0 5.08 90) (size 1.7 1.7) (drill 1) (layers "*.Cu" "*.Mask") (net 6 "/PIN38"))
  (pad "4" thru_hole oval (at 0 7.62 90) (size 1.7 1.7) (drill 1) (layers "*.Cu" "*.Mask") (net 8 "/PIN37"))
  (pad "5" thru_hole oval (at 0 10.16 90) (size 1.7 1.7) (drill 1) (layers "*.Cu" "*.Mask") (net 10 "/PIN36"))
  (pad "6" thru_hole oval (at 0 12.7 90) (size 1.7 1.7) (drill 1) (layers "*.Cu" "*.Mask") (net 12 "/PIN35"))
  (pad "7" thru_hole oval (at 0 15.24 90) (size 1.7 1.7) (drill 1) (layers "*.Cu" "*.Mask") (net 14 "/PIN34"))
  (pad "8" thru_hole oval (at 0 17.78 90) (size 1.7 1.7) (drill 1) (layers "*.Cu" "*.Mask") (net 16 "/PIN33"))
  (pad "9" thru_hole oval (at 0 20.32 90) (size 1.7 1.7) (drill 1) (layers "*.Cu" "*.Mask") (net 18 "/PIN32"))
  (pad "10" thru_hole oval (at 0 22.86 90) (size 1.7 1.7) (drill 1) (layers "*.Cu" "*.Mask") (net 20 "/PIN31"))
  (pad "11" thru_hole oval (at 0 25.4 90) (size 1.7 1.7) (drill 1) (layers "*.Cu" "*.Mask") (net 22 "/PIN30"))
  (pad "12" thru_hole oval (at 0 27.94 90) (size 1.7 1.7) (drill 1) (layers "*.Cu" "*.Mask") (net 24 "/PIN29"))
  (pad "13" thru_hole oval (at 0 30.48 90) (size 1.7 1.7) (drill 1) (layers "*.Cu" "*.Mask") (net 26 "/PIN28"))
  (pad "14" thru_hole oval (at 0 33.02 90) (size 1.7 1.7) (drill 1) (layers "*.Cu" "*.Mask") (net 28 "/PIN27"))
  (pad "15" thru_hole oval (at 0 35.56 90) (size 1.7 1.7) (drill 1) (layers "*.Cu" "*.Mask") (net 30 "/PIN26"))
  (pad "16" thru_hole oval (at 0 38.1 90) (size 1.7 1.7) (drill 1) (layers "*.Cu" "*.Mask") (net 32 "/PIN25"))
  (pad "17" thru_hole oval (at 0 40.64 90) (size 1.7 1.7) (drill 1) (layers "*.Cu" "*.Mask") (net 34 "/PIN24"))
  (pad "18" thru_hole oval (at 0 43.18 90) (size 1.7 1.7) (drill 1) (layers "*.Cu" "*.Mask") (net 36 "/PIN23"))
  (pad "19" thru_hole oval (at 0 45.72 90) (size 1.7 1.7) (drill 1) (layers "*.Cu" "*.Mask") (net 38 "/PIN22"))
  (pad "20" thru_hole oval (at 0 48.26 90) (size 1.7 1.7) (drill 1) (layers "*.Cu" "*.Mask") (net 40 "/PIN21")))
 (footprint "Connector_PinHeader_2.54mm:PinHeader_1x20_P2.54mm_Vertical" (layer "F.Cu") (at 125.095 99.175 90)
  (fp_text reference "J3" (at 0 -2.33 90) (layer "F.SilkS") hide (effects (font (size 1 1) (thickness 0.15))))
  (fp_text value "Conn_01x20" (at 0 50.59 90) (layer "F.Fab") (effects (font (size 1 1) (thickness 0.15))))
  (pad "1" thru_hole circle (at 0 0 90) (size 1.7 1.7) (drill 1) (layers "*.Cu" "*.Mask") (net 1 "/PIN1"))
  (pad "2" thru_hole oval (at 0 2.54 90) (size 1.7 1.7) (drill 1) (layers "*.Cu" "*.Mask") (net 3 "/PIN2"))
  (pad "3" thru_hole oval (at 0 5.08 90) (size 1.7 1.7) (drill 1) (layers "*.Cu" "*.Mask") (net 5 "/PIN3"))
  (pad "4" thru_hole oval (at 0 7.62 90) (size 1.7 1.7) (drill 1) (layers "*.Cu" "*.Mask") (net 7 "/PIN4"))
  (pad "5" thru_hole oval (at 0 10.16 90) (size 1.7 1.7) (drill 1) (layers "*.Cu" "*.Mask") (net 9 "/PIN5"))
  (pad "6" thru_hole oval (at 0 12.7 90) (size 1.7 1.7) (drill 1) (layers "*.Cu" "*.Mask") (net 11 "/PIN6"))
  (pad "7" thru_hole oval (at 0 15.24 90) (size 1.7 1.7) (drill 1) (layers "*.Cu" "*.Mask") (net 13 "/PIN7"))
  (pad "8" thru_hole oval (at 0 17.78 90) (size 1.7 1.7) (drill 1) (layers "*.Cu" "*.Mask") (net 15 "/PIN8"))
  (pad "9" thru_hole oval (at 0 20.32 90) (size 1.7 1.7) (drill 1) (layers "*.Cu" "*.Mask") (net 17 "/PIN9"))
  (pad "10" thru_hole oval (at 0 22.86 90) (size 1.7 1.7) (drill 1) (layers "*.Cu" "*.Mask") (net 19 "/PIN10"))
  (pad "11" thru_hole oval (at 0 25.4 90) (size 1.7 1.7) (drill 1) (layers "*.Cu" "*.Mask") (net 21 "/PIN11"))
  (pad "12" thru_hole oval (at 0 27.94 90) (size 1.7 1.7) (drill 1) (layers "*.Cu" "*.Mask") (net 23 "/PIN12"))
  (pad "13" thru_hole oval (at 0 30.48 90) (size 1.7 1.7) (drill 1) (layers "*.Cu" "*.Mask") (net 25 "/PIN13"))
  (pad "14" thru_hole oval (at 0 33.02 90) (size 1.7 1.7) (drill 1) (layers "*.Cu" "*.Mask") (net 27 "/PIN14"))
  (pad "15" thru_hole oval (at 0 35.56 90) (size 1.7 1.7) (drill 1) (layers "*.Cu" "*.Mask") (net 29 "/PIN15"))
  (pad "16" thru_hole oval (at 0 38.1 90) (size 1.7 1.7) (drill 1) (layers "*.Cu" "*.Mask") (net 31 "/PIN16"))
  (pad "17" thru_hole oval (at 0 40.64 90) (size 1.7 1.7) (drill 1) (layers "*.Cu" "*.Mask") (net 33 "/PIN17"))
  (pad "18" thru_hole oval (at 0 43.18 90) (size 1.7 1.7) (drill 1) (layers "*.Cu" "*.Mask") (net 35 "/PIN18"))
  (pad "19" thru_hole oval (at 0 45.72 90) (size 1.7 1.7) (drill 1) (layers "*.Cu" "*.Mask") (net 37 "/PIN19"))
  (pad "20" thru_hole oval (at 0 48.26 90) (size 1.7 1.7) (drill 1) (layers "*.Cu" "*.Mask") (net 39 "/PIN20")))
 (gr_circle (center 126.24485 100.681893) (end 126.55407 100.681893) (stroke (width 0.2) (type solid)) (fill solid) (layer "F.Cu"))
 (gr_rect (start 123.825 87.63) (end 174.625 102.87) (stroke (width 0.1) (type solid)) (fill none) (layer "Edge.Cuts"))
 (segment (start 125.095 96.635) (end 125.095 102.12) (width 0.4) (layer "B.Cu") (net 1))
 (segment (start 127.635 96.635) (end 127.635 102.12) (width 0.4) (layer "B.Cu") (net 3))
 (segment (start 130.175 96.635) (end 130.175 102.12) (width 0.4) (layer "B.Cu") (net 5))
 (segment (start 132.715 96.635) (end 132.715 102.12) (width 0.4) (layer "B.Cu") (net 7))
 (segment (start 135.255 96.635) (end 135.255 102.12) (width 0.4) (layer "B.Cu") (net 9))
 (segment (start 137.795 96.635) (end 137.795 102.12) (width 0.4) (layer "B.Cu") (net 11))
 (segment (start 140.335 96.635) (end 140.335 102.12) (width 0.4) (layer "B.Cu") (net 13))
 (segment (start 142.875 96.635) (end 142.875 102.12) (width 0.4) (layer "B.Cu") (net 15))
 (segment (start 145.415 96.635) (end 145.415 102.12) (width 0.4) (layer "B.Cu") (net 17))
 (segment (start 147.955 96.635) (end 147.955 102.12) (width 0.4) (layer "B.Cu") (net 19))
 (segment (start 150.495 96.635) (end 150.495 102.12) (width 0.4) (layer "B.Cu") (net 21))
 (segment (start 153.035 96.635) (end 153.035 102.12) (width 0.4) (layer "B.Cu") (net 23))
 (segment (start 155.575 96.635) (end 155.575 102.12) (width 0.4) (layer "B.Cu") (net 25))
 (segment (start 158.115 96.635) (end 158.115 102.12) (width 0.4) (layer "B.Cu") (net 27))
 (segment (start 163.195 96.635) (end 163.195 102.12) (width 0.4) (layer "B.Cu") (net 31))
 (segment (start 165.735 96.635) (end 165.735 102.12) (width 0.4) (layer "B.Cu") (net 33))
 (segment (start 168.275 96.635) (end 168.275 102.12) (width 0.4) (layer "B.Cu") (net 35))
 (segment (start 170.815 96.635) (end 170.815 102.12) (width 0.4) (layer "B.Cu") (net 37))
 (segment (start 173.355 96.635) (end 173.355 102.12) (width 0.4) (layer "B.Cu") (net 39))
 (segment (start 173.355 88.38) (end 173.355 94.095) (width 0.4) (layer "B.Cu") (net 40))
 (segment (start 170.815 88.38) (end 170.815 94.095) (width 0.4) (layer "B.Cu") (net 38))
 (segment (start 168.275 88.38) (end 168.275 94.095) (width 0.4) (layer "B.Cu") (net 36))
 (segment (start 165.735 88.38) (end 165.735 94.095) (width 0.4) (layer "B.Cu") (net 34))
 (segment (start 163.195 88.38) (end 163.195 94.095) (width 0.4) (layer "B.Cu") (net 32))
 (segment (start 160.655 88.38) (end 160.655 94.095) (width 0.4) (layer "B.Cu") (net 30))
 (segment (start 158.115 88.38) (end 158.115 94.095) (width 0.4) (layer "B.Cu") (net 28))
 (segment (start 155.575 88.38) (end 155.575 94.095) (width 0.4) (layer "B.Cu") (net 26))
 (segment (start 153.035 88.38) (end 153.035 94.095) (width 0.4) (layer "B.Cu") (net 24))
 (segment (start 150.495 88.38) (end 150.495 94.095) (width 0.4) (layer "B.Cu") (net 22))
 (segment (start 147.955 88.38) (end 147.955 94.095) (width 0.4) (layer "B.Cu") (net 20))
 (segment (start 145.415 88.38) (end 145.415 94.095) (width 0.4) (layer "B.Cu") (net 18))
 (segment (start 142.875 88.38) (end 142.875 94.095) (width 0.4) (layer "B.Cu") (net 16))
 (segment (start 140.335 88.38) (end 140.335 94.095) (width 0.4) (layer "B.Cu") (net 14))
 (segment (start 137.795 88.38) (end 137.795 94.095) (width 0.4) (layer "B.Cu") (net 12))
 (segment (start 135.255 88.38) (end 135.255 94.095) (width 0.4) (layer "B.Cu") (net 10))
 (segment (start 132.715 88.38) (end 132.715 94.095) (width 0.4) (layer "B.Cu") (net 8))
 (segment (start 130.175 88.38) (end 130.175 94.095) (width 0.4) (layer "B.Cu") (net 6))
 (segment (start 127.635 88.38) (end 127.635 94.095) (width 0.4) (layer "B.Cu") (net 4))
 (segment (start 125.095 88.38) (end 125.095 94.095) (width 0.4) (layer "B.Cu") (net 2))
 (segment (start 160.655 96.635) (end 160.655 102.12) (width 0.4) (layer "B.Cu") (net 29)))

